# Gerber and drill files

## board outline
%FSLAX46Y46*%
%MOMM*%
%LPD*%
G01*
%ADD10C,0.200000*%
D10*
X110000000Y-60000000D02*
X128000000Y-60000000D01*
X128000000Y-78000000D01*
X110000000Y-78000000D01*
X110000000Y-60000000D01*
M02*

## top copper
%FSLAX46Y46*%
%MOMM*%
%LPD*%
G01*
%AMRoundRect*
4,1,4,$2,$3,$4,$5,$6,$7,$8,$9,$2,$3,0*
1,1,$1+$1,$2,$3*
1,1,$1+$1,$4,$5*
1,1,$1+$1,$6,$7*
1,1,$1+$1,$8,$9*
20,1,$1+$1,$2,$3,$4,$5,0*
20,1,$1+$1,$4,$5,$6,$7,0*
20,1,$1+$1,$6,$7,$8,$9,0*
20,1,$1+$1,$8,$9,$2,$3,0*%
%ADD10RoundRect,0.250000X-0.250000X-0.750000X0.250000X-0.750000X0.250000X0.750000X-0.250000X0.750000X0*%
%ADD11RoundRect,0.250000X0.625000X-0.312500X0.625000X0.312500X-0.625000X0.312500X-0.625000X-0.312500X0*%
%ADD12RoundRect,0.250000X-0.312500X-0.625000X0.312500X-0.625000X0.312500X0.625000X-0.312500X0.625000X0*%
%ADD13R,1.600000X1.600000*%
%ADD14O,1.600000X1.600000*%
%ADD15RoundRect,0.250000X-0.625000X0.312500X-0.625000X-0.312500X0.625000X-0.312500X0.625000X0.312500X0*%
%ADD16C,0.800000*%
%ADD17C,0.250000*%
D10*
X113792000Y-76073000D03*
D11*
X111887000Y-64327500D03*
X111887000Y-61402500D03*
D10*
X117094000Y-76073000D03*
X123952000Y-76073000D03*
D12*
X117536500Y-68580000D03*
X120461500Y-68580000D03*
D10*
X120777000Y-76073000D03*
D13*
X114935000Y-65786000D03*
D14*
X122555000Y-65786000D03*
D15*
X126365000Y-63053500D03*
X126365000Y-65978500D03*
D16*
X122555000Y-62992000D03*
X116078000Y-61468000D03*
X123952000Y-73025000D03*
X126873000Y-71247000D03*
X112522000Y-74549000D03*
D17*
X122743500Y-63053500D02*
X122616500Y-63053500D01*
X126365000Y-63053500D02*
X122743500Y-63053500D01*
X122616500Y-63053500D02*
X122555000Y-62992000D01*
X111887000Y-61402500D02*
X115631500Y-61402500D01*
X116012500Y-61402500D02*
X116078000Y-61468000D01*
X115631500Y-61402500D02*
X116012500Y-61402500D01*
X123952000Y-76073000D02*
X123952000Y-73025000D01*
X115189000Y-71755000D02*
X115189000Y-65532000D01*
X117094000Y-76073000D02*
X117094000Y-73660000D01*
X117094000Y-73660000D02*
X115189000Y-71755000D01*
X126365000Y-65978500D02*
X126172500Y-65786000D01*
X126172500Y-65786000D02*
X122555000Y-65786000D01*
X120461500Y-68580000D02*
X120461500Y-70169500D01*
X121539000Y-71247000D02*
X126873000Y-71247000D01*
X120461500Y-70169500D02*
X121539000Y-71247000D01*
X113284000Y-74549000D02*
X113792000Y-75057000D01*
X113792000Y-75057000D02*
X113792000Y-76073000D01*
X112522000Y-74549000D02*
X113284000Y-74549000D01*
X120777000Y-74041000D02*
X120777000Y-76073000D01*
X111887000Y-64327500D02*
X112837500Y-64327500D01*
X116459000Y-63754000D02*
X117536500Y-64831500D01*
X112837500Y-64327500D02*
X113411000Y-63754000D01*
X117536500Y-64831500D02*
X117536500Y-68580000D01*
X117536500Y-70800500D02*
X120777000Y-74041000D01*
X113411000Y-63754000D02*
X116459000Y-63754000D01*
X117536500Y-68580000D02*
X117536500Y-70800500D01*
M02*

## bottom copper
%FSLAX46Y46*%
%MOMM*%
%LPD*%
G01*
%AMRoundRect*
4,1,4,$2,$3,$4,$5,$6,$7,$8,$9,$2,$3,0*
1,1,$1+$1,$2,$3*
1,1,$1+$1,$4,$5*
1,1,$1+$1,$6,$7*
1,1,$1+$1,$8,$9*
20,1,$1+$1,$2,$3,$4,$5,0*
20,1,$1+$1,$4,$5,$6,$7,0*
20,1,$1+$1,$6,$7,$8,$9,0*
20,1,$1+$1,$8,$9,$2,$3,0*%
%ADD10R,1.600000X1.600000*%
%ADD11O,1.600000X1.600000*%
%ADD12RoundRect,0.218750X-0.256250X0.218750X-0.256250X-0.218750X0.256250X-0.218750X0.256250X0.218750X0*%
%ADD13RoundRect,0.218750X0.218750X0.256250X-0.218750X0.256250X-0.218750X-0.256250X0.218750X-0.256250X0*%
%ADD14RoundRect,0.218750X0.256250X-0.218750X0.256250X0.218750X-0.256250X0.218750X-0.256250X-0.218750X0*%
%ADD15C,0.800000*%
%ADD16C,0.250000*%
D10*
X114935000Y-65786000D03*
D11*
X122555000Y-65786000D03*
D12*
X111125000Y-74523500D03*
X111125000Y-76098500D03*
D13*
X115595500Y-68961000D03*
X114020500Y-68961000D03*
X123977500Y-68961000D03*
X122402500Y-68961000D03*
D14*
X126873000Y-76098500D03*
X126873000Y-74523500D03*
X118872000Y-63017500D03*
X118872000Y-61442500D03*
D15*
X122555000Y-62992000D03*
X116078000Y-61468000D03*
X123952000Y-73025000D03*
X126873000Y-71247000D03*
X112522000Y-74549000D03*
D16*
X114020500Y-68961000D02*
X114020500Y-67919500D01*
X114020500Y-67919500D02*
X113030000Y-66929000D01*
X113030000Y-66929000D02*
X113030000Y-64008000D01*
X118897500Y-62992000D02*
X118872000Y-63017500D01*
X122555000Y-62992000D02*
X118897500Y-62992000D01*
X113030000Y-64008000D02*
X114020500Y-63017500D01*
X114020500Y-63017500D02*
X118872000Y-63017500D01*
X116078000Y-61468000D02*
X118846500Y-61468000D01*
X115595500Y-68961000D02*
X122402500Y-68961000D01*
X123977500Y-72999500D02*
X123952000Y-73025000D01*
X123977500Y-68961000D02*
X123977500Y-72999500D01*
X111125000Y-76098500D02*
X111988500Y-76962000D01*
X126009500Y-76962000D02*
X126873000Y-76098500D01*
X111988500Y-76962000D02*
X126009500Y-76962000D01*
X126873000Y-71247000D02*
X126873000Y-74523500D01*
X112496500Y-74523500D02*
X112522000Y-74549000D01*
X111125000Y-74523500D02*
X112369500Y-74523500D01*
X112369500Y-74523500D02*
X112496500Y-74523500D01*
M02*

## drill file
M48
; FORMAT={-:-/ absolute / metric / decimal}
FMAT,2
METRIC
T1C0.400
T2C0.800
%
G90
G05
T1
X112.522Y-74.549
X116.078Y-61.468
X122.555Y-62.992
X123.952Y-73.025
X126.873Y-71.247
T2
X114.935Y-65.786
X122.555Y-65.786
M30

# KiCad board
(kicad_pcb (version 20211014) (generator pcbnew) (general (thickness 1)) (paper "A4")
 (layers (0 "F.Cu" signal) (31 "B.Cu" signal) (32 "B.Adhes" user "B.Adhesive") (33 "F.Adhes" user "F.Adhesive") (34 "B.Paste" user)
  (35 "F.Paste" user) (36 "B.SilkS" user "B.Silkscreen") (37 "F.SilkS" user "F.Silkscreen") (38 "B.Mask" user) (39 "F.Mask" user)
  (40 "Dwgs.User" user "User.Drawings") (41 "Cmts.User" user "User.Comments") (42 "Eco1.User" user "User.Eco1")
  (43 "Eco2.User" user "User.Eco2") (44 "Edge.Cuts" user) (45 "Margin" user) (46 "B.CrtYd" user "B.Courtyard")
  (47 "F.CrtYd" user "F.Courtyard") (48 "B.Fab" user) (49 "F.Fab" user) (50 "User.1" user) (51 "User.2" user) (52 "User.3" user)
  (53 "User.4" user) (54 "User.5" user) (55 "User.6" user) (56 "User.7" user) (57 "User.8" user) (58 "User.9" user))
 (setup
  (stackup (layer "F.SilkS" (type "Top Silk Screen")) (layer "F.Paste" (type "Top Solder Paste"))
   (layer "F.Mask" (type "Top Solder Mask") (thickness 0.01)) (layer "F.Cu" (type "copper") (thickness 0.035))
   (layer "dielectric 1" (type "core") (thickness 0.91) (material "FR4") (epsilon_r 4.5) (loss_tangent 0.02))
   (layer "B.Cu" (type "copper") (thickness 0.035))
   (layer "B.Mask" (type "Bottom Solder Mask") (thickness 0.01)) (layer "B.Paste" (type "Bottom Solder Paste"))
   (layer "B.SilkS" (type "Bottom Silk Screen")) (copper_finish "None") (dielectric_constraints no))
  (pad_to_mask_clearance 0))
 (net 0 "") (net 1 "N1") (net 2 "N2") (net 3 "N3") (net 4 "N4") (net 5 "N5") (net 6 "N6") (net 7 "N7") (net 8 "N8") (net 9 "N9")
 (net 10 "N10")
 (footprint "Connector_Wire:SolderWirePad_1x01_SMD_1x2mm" (layer "F.Cu") (at 113.792 76.073)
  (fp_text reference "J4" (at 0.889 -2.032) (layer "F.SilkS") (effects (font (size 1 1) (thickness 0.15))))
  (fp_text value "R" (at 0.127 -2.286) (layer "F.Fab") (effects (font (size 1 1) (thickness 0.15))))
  (pad "1" smd roundrect (at 0 0) (size 1 2) (layers "F.Cu" "B.Paste" "F.Mask") (roundrect_rratio 0.25) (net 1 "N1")))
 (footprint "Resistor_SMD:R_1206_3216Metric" (layer "F.Cu") (at 111.887 62.865 90)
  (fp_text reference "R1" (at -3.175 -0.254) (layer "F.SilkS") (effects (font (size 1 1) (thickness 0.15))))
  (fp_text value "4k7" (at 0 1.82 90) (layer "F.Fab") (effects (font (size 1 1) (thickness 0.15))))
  (pad "1" smd roundrect (at -1.4625 0 90) (size 1.125 1.75) (layers "F.Cu" "F.Paste" "F.Mask") (roundrect_rratio 0.2222222222) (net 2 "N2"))
  (pad "2" smd roundrect (at 1.4625 0 90) (size 1.125 1.75) (layers "F.Cu" "F.Paste" "F.Mask") (roundrect_rratio 0.2222222222) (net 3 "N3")))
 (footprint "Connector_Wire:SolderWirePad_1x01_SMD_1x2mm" (layer "F.Cu") (at 117.094 76.073)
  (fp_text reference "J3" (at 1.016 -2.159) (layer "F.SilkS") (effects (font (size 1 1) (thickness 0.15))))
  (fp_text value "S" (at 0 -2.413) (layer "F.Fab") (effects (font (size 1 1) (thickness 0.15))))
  (pad "1" smd roundrect (at 0 0) (size 1 2) (layers "F.Cu" "F.Paste" "F.Mask") (roundrect_rratio 0.25) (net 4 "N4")))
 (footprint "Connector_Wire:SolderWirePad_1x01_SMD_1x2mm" (layer "F.Cu") (at 123.952 76.073)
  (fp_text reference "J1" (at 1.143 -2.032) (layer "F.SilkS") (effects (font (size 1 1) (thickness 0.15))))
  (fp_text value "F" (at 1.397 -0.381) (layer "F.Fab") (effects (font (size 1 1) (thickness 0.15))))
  (pad "1" smd roundrect (at 0 0) (size 1 2) (layers "F.Cu" "F.SilkS" "F.Mask") (roundrect_rratio 0.25) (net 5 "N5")))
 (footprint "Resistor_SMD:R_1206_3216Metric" (layer "F.Cu") (at 118.999 68.58)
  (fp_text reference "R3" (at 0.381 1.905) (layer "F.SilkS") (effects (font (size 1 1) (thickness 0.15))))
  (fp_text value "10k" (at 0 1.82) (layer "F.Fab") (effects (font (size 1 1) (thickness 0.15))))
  (pad "1" smd roundrect (at -1.4625 0) (size 1.125 1.75) (layers "F.Cu" "F.Paste" "F.Mask") (roundrect_rratio 0.2222222222) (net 2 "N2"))
  (pad "2" smd roundrect (at 1.4625 0) (size 1.125 1.75) (layers "F.Cu" "F.Paste" "F.Mask") (roundrect_rratio 0.2222222222) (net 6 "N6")))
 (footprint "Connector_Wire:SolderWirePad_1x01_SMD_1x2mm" (layer "F.Cu") (at 120.777 76.073)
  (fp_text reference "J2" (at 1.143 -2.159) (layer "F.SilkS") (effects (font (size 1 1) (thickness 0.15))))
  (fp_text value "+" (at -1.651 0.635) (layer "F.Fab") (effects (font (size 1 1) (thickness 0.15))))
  (pad "1" smd roundrect (at 0 0) (size 1 2) (layers "F.Cu" "F.Paste" "F.Mask") (roundrect_rratio 0.25) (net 2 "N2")))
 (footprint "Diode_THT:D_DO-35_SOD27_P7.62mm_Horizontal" (layer "F.Cu") (at 114.935 65.786)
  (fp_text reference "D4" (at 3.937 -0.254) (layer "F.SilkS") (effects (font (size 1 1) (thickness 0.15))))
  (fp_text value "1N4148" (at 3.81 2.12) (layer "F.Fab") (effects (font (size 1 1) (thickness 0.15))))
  (pad "1" thru_hole rect (at 0 0) (size 1.6 1.6) (drill 0.8) (layers *.Cu *.Mask) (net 4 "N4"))
  (pad "2" thru_hole oval (at 7.62 0) (size 1.6 1.6) (drill 0.8) (layers *.Cu *.Mask) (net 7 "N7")))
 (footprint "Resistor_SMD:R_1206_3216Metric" (layer "F.Cu") (at 126.365 64.516 -90)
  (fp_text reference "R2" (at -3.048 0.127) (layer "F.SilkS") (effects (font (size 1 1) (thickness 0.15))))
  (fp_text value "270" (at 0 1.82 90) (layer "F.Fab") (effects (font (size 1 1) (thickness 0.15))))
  (pad "1" smd roundrect (at -1.4625 0 270) (size 1.125 1.75) (layers "F.Cu" "F.Paste" "F.Mask") (roundrect_rratio 0.2222222222)
   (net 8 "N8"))
  (pad "2" smd roundrect (at 1.4625 0 270) (size 1.125 1.75) (layers "F.Cu" "F.Paste" "F.Mask") (roundrect_rratio 0.2222222222) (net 7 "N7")))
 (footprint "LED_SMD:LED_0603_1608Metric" (layer "B.Cu") (at 111.125 75.311 -90)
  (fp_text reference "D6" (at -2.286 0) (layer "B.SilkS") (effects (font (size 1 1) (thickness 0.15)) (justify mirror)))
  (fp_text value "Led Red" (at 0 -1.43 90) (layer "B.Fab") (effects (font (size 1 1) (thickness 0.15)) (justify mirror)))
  (pad "1" smd roundrect (at -0.7875 0 270) (size 0.875 0.95) (layers "B.Cu" "B.Paste" "B.Mask") (roundrect_rratio 0.25) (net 1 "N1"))
  (pad "2" smd roundrect (at 0.7875 0 270) (size 0.875 0.95) (layers "B.Cu" "B.Paste" "B.Mask") (roundrect_rratio 0.25) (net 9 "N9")))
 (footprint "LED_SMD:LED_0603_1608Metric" (layer "B.Cu") (at 114.808 68.961 180)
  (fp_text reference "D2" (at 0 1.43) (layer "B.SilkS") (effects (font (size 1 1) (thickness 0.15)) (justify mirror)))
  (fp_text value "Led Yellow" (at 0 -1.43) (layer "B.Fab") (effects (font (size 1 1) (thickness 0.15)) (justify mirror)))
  (pad "1" smd roundrect (at -0.7875 0 180) (size 0.875 0.95) (layers "B.Cu" "B.Paste" "B.Mask") (roundrect_rratio 0.25) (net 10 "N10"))
  (pad "2" smd roundrect (at 0.7875 0 180) (size 0.875 0.95) (layers "B.Cu" "B.Paste" "B.Mask") (roundrect_rratio 0.25) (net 8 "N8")))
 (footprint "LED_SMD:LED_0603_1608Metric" (layer "B.Cu") (at 123.19 68.961 180)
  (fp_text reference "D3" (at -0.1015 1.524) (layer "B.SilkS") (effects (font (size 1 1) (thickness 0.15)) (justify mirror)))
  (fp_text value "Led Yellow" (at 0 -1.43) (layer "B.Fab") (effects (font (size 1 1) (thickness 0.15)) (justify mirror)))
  (pad "1" smd roundrect (at -0.7875 0 180) (size 0.875 0.95) (layers "B.Cu" "B.Paste" "B.Mask") (roundrect_rratio 0.25) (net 5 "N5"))
  (pad "2" smd roundrect (at 0.7875 0 180) (size 0.875 0.95) (layers "B.Cu" "B.Paste" "B.Mask") (roundrect_rratio 0.25) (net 10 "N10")))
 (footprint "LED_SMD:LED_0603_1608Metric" (layer "B.Cu") (at 126.873 75.311 90)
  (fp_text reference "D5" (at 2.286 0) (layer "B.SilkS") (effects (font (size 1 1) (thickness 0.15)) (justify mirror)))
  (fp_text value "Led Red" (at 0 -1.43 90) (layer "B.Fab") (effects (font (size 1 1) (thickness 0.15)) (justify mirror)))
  (pad "1" smd roundrect (at -0.7875 0 90) (size 0.875 0.95) (layers "B.Cu" "B.Paste" "B.Mask") (roundrect_rratio 0.25) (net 9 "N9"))
  (pad "2" smd roundrect (at 0.7875 0 90) (size 0.875 0.95) (layers "B.Cu" "B.Paste" "B.Mask") (roundrect_rratio 0.25) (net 6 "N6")))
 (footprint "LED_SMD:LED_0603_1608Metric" (layer "B.Cu") (at 118.872 62.23 90)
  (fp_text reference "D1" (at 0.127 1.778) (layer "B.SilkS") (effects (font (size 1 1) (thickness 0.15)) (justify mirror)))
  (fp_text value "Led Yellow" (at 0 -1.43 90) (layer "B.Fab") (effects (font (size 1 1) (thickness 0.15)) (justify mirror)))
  (pad "1" smd roundrect (at -0.7875 0 90) (size 0.875 0.95) (layers "B.Cu" "B.Paste" "B.Mask") (roundrect_rratio 0.25) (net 8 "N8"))
  (pad "2" smd roundrect (at 0.7875 0 90) (size 0.875 0.95) (layers "B.Cu" "B.Paste" "B.Mask") (roundrect_rratio 0.25) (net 3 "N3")))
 (gr_rect locked (start 110 60) (end 128 78) (layer "Edge.Cuts") (width 0.2) (fill none))
 (segment (start 122.7435 63.0535) (end 122.6165 63.0535) (width 0.25) (layer "F.Cu") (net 8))
 (segment (start 126.365 63.0535) (end 122.7435 63.0535) (width 0.25) (layer "F.Cu") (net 8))
 (segment (start 122.6165 63.0535) (end 122.555 62.992) (width 0.25) (layer "F.Cu") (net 8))
 (via (at 122.555 62.992) (size 0.8) (drill 0.4) (layers "F.Cu" "B.Cu") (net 8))
 (segment (start 114.0205 68.961) (end 114.0205 67.9195) (width 0.25) (layer "B.Cu") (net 8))
 (segment (start 114.0205 67.9195) (end 113.03 66.929) (width 0.25) (layer "B.Cu") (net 8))
 (segment (start 113.03 66.929) (end 113.03 64.008) (width 0.25) (layer "B.Cu") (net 8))
 (segment (start 118.8975 62.992) (end 118.872 63.0175) (width 0.25) (layer "B.Cu") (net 8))
 (segment (start 122.555 62.992) (end 118.8975 62.992) (width 0.25) (layer "B.Cu") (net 8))
 (segment (start 113.03 64.008) (end 114.0205 63.0175) (width 0.25) (layer "B.Cu") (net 8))
 (segment (start 114.0205 63.0175) (end 118.872 63.0175) (width 0.25) (layer "B.Cu") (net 8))
 (segment (start 111.887 61.4025) (end 115.6315 61.4025) (width 0.25) (layer "F.Cu") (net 3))
 (segment (start 116.0125 61.4025) (end 116.078 61.468) (width 0.25) (layer "F.Cu") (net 3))
 (segment (start 115.6315 61.4025) (end 116.0125 61.4025) (width 0.25) (layer "F.Cu") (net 3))
 (via (at 116.078 61.468) (size 0.8) (drill 0.4) (layers "F.Cu" "B.Cu") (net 3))
 (segment (start 116.078 61.468) (end 118.8465 61.468) (width 0.25) (layer "B.Cu") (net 3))
 (segment (start 115.5955 68.961) (end 122.4025 68.961) (width 0.25) (layer "B.Cu") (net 10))
 (segment (start 123.952 76.073) (end 123.952 73.025) (width 0.25) (layer "F.Cu") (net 5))
 (via (at 123.952 73.025) (size 0.8) (drill 0.4) (layers "F.Cu" "B.Cu") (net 5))
 (segment (start 123.9775 72.9995) (end 123.952 73.025) (width 0.25) (layer "B.Cu") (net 5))
 (segment (start 123.9775 68.961) (end 123.9775 72.9995) (width 0.25) (layer "B.Cu") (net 5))
 (segment (start 115.189 71.755) (end 115.189 65.532) (width 0.25) (layer "F.Cu") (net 4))
 (segment (start 117.094 76.073) (end 117.094 73.66) (width 0.25) (layer "F.Cu") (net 4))
 (segment (start 117.094 73.66) (end 115.189 71.755) (width 0.25) (layer "F.Cu") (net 4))
 (segment (start 126.365 65.9785) (end 126.1725 65.786) (width 0.25) (layer "F.Cu") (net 7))
 (segment (start 126.1725 65.786) (end 122.555 65.786) (width 0.25) (layer "F.Cu") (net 7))
 (segment (start 111.125 76.0985) (end 111.9885 76.962) (width 0.25) (layer "B.Cu") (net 9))
 (segment (start 126.0095 76.962) (end 126.873 76.0985) (width 0.25) (layer "B.Cu") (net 9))
 (segment (start 111.9885 76.962) (end 126.0095 76.962) (width 0.25) (layer "B.Cu") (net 9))
 (segment (start 120.4615 68.58) (end 120.4615 70.1695) (width 0.25) (layer "F.Cu") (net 6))
 (segment (start 121.539 71.247) (end 126.873 71.247) (width 0.25) (layer "F.Cu") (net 6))
 (segment (start 120.4615 70.1695) (end 121.539 71.247) (width 0.25) (layer "F.Cu") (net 6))
 (via (at 126.873 71.247) (size 0.8) (drill 0.4) (layers "F.Cu" "B.Cu") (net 6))
 (segment (start 126.873 71.247) (end 126.873 74.5235) (width 0.25) (layer "B.Cu") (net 6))
 (segment (start 113.284 74.549) (end 113.792 75.057) (width 0.25) (layer "F.Cu") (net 1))
 (segment (start 113.792 75.057) (end 113.792 76.073) (width 0.25) (layer "F.Cu") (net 1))
 (segment (start 112.522 74.549) (end 113.284 74.549) (width 0.25) (layer "F.Cu") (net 1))
 (via (at 112.522 74.549) (size 0.8) (drill 0.4) (layers "F.Cu" "B.Cu") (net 1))
 (segment (start 112.4965 74.5235) (end 112.522 74.549) (width 0.25) (layer "B.Cu") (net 1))
 (segment (start 111.125 74.5235) (end 112.3695 74.5235) (width 0.25) (layer "B.Cu") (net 1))
 (segment (start 112.3695 74.5235) (end 112.4965 74.5235) (width 0.25) (layer "B.Cu") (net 1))
 (segment (start 120.777 74.041) (end 120.777 76.073) (width 0.25) (layer "F.Cu") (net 2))
 (segment (start 111.887 64.3275) (end 112.8375 64.3275) (width 0.25) (layer "F.Cu") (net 2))
 (segment (start 116.459 63.754) (end 117.5365 64.8315) (width 0.25) (layer "F.Cu") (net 2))
 (segment (start 112.8375 64.3275) (end 113.411 63.754) (width 0.25) (layer "F.Cu") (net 2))
 (segment (start 117.5365 64.8315) (end 117.5365 68.58) (width 0.25) (layer "F.Cu") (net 2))
 (segment (start 117.5365 70.8005) (end 120.777 74.041) (width 0.25) (layer "F.Cu") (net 2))
 (segment (start 113.411 63.754) (end 116.459 63.754) (width 0.25) (layer "F.Cu") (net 2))
 (segment (start 117.5365 68.58) (end 117.5365 70.8005) (width 0.25) (layer "F.Cu") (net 2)))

